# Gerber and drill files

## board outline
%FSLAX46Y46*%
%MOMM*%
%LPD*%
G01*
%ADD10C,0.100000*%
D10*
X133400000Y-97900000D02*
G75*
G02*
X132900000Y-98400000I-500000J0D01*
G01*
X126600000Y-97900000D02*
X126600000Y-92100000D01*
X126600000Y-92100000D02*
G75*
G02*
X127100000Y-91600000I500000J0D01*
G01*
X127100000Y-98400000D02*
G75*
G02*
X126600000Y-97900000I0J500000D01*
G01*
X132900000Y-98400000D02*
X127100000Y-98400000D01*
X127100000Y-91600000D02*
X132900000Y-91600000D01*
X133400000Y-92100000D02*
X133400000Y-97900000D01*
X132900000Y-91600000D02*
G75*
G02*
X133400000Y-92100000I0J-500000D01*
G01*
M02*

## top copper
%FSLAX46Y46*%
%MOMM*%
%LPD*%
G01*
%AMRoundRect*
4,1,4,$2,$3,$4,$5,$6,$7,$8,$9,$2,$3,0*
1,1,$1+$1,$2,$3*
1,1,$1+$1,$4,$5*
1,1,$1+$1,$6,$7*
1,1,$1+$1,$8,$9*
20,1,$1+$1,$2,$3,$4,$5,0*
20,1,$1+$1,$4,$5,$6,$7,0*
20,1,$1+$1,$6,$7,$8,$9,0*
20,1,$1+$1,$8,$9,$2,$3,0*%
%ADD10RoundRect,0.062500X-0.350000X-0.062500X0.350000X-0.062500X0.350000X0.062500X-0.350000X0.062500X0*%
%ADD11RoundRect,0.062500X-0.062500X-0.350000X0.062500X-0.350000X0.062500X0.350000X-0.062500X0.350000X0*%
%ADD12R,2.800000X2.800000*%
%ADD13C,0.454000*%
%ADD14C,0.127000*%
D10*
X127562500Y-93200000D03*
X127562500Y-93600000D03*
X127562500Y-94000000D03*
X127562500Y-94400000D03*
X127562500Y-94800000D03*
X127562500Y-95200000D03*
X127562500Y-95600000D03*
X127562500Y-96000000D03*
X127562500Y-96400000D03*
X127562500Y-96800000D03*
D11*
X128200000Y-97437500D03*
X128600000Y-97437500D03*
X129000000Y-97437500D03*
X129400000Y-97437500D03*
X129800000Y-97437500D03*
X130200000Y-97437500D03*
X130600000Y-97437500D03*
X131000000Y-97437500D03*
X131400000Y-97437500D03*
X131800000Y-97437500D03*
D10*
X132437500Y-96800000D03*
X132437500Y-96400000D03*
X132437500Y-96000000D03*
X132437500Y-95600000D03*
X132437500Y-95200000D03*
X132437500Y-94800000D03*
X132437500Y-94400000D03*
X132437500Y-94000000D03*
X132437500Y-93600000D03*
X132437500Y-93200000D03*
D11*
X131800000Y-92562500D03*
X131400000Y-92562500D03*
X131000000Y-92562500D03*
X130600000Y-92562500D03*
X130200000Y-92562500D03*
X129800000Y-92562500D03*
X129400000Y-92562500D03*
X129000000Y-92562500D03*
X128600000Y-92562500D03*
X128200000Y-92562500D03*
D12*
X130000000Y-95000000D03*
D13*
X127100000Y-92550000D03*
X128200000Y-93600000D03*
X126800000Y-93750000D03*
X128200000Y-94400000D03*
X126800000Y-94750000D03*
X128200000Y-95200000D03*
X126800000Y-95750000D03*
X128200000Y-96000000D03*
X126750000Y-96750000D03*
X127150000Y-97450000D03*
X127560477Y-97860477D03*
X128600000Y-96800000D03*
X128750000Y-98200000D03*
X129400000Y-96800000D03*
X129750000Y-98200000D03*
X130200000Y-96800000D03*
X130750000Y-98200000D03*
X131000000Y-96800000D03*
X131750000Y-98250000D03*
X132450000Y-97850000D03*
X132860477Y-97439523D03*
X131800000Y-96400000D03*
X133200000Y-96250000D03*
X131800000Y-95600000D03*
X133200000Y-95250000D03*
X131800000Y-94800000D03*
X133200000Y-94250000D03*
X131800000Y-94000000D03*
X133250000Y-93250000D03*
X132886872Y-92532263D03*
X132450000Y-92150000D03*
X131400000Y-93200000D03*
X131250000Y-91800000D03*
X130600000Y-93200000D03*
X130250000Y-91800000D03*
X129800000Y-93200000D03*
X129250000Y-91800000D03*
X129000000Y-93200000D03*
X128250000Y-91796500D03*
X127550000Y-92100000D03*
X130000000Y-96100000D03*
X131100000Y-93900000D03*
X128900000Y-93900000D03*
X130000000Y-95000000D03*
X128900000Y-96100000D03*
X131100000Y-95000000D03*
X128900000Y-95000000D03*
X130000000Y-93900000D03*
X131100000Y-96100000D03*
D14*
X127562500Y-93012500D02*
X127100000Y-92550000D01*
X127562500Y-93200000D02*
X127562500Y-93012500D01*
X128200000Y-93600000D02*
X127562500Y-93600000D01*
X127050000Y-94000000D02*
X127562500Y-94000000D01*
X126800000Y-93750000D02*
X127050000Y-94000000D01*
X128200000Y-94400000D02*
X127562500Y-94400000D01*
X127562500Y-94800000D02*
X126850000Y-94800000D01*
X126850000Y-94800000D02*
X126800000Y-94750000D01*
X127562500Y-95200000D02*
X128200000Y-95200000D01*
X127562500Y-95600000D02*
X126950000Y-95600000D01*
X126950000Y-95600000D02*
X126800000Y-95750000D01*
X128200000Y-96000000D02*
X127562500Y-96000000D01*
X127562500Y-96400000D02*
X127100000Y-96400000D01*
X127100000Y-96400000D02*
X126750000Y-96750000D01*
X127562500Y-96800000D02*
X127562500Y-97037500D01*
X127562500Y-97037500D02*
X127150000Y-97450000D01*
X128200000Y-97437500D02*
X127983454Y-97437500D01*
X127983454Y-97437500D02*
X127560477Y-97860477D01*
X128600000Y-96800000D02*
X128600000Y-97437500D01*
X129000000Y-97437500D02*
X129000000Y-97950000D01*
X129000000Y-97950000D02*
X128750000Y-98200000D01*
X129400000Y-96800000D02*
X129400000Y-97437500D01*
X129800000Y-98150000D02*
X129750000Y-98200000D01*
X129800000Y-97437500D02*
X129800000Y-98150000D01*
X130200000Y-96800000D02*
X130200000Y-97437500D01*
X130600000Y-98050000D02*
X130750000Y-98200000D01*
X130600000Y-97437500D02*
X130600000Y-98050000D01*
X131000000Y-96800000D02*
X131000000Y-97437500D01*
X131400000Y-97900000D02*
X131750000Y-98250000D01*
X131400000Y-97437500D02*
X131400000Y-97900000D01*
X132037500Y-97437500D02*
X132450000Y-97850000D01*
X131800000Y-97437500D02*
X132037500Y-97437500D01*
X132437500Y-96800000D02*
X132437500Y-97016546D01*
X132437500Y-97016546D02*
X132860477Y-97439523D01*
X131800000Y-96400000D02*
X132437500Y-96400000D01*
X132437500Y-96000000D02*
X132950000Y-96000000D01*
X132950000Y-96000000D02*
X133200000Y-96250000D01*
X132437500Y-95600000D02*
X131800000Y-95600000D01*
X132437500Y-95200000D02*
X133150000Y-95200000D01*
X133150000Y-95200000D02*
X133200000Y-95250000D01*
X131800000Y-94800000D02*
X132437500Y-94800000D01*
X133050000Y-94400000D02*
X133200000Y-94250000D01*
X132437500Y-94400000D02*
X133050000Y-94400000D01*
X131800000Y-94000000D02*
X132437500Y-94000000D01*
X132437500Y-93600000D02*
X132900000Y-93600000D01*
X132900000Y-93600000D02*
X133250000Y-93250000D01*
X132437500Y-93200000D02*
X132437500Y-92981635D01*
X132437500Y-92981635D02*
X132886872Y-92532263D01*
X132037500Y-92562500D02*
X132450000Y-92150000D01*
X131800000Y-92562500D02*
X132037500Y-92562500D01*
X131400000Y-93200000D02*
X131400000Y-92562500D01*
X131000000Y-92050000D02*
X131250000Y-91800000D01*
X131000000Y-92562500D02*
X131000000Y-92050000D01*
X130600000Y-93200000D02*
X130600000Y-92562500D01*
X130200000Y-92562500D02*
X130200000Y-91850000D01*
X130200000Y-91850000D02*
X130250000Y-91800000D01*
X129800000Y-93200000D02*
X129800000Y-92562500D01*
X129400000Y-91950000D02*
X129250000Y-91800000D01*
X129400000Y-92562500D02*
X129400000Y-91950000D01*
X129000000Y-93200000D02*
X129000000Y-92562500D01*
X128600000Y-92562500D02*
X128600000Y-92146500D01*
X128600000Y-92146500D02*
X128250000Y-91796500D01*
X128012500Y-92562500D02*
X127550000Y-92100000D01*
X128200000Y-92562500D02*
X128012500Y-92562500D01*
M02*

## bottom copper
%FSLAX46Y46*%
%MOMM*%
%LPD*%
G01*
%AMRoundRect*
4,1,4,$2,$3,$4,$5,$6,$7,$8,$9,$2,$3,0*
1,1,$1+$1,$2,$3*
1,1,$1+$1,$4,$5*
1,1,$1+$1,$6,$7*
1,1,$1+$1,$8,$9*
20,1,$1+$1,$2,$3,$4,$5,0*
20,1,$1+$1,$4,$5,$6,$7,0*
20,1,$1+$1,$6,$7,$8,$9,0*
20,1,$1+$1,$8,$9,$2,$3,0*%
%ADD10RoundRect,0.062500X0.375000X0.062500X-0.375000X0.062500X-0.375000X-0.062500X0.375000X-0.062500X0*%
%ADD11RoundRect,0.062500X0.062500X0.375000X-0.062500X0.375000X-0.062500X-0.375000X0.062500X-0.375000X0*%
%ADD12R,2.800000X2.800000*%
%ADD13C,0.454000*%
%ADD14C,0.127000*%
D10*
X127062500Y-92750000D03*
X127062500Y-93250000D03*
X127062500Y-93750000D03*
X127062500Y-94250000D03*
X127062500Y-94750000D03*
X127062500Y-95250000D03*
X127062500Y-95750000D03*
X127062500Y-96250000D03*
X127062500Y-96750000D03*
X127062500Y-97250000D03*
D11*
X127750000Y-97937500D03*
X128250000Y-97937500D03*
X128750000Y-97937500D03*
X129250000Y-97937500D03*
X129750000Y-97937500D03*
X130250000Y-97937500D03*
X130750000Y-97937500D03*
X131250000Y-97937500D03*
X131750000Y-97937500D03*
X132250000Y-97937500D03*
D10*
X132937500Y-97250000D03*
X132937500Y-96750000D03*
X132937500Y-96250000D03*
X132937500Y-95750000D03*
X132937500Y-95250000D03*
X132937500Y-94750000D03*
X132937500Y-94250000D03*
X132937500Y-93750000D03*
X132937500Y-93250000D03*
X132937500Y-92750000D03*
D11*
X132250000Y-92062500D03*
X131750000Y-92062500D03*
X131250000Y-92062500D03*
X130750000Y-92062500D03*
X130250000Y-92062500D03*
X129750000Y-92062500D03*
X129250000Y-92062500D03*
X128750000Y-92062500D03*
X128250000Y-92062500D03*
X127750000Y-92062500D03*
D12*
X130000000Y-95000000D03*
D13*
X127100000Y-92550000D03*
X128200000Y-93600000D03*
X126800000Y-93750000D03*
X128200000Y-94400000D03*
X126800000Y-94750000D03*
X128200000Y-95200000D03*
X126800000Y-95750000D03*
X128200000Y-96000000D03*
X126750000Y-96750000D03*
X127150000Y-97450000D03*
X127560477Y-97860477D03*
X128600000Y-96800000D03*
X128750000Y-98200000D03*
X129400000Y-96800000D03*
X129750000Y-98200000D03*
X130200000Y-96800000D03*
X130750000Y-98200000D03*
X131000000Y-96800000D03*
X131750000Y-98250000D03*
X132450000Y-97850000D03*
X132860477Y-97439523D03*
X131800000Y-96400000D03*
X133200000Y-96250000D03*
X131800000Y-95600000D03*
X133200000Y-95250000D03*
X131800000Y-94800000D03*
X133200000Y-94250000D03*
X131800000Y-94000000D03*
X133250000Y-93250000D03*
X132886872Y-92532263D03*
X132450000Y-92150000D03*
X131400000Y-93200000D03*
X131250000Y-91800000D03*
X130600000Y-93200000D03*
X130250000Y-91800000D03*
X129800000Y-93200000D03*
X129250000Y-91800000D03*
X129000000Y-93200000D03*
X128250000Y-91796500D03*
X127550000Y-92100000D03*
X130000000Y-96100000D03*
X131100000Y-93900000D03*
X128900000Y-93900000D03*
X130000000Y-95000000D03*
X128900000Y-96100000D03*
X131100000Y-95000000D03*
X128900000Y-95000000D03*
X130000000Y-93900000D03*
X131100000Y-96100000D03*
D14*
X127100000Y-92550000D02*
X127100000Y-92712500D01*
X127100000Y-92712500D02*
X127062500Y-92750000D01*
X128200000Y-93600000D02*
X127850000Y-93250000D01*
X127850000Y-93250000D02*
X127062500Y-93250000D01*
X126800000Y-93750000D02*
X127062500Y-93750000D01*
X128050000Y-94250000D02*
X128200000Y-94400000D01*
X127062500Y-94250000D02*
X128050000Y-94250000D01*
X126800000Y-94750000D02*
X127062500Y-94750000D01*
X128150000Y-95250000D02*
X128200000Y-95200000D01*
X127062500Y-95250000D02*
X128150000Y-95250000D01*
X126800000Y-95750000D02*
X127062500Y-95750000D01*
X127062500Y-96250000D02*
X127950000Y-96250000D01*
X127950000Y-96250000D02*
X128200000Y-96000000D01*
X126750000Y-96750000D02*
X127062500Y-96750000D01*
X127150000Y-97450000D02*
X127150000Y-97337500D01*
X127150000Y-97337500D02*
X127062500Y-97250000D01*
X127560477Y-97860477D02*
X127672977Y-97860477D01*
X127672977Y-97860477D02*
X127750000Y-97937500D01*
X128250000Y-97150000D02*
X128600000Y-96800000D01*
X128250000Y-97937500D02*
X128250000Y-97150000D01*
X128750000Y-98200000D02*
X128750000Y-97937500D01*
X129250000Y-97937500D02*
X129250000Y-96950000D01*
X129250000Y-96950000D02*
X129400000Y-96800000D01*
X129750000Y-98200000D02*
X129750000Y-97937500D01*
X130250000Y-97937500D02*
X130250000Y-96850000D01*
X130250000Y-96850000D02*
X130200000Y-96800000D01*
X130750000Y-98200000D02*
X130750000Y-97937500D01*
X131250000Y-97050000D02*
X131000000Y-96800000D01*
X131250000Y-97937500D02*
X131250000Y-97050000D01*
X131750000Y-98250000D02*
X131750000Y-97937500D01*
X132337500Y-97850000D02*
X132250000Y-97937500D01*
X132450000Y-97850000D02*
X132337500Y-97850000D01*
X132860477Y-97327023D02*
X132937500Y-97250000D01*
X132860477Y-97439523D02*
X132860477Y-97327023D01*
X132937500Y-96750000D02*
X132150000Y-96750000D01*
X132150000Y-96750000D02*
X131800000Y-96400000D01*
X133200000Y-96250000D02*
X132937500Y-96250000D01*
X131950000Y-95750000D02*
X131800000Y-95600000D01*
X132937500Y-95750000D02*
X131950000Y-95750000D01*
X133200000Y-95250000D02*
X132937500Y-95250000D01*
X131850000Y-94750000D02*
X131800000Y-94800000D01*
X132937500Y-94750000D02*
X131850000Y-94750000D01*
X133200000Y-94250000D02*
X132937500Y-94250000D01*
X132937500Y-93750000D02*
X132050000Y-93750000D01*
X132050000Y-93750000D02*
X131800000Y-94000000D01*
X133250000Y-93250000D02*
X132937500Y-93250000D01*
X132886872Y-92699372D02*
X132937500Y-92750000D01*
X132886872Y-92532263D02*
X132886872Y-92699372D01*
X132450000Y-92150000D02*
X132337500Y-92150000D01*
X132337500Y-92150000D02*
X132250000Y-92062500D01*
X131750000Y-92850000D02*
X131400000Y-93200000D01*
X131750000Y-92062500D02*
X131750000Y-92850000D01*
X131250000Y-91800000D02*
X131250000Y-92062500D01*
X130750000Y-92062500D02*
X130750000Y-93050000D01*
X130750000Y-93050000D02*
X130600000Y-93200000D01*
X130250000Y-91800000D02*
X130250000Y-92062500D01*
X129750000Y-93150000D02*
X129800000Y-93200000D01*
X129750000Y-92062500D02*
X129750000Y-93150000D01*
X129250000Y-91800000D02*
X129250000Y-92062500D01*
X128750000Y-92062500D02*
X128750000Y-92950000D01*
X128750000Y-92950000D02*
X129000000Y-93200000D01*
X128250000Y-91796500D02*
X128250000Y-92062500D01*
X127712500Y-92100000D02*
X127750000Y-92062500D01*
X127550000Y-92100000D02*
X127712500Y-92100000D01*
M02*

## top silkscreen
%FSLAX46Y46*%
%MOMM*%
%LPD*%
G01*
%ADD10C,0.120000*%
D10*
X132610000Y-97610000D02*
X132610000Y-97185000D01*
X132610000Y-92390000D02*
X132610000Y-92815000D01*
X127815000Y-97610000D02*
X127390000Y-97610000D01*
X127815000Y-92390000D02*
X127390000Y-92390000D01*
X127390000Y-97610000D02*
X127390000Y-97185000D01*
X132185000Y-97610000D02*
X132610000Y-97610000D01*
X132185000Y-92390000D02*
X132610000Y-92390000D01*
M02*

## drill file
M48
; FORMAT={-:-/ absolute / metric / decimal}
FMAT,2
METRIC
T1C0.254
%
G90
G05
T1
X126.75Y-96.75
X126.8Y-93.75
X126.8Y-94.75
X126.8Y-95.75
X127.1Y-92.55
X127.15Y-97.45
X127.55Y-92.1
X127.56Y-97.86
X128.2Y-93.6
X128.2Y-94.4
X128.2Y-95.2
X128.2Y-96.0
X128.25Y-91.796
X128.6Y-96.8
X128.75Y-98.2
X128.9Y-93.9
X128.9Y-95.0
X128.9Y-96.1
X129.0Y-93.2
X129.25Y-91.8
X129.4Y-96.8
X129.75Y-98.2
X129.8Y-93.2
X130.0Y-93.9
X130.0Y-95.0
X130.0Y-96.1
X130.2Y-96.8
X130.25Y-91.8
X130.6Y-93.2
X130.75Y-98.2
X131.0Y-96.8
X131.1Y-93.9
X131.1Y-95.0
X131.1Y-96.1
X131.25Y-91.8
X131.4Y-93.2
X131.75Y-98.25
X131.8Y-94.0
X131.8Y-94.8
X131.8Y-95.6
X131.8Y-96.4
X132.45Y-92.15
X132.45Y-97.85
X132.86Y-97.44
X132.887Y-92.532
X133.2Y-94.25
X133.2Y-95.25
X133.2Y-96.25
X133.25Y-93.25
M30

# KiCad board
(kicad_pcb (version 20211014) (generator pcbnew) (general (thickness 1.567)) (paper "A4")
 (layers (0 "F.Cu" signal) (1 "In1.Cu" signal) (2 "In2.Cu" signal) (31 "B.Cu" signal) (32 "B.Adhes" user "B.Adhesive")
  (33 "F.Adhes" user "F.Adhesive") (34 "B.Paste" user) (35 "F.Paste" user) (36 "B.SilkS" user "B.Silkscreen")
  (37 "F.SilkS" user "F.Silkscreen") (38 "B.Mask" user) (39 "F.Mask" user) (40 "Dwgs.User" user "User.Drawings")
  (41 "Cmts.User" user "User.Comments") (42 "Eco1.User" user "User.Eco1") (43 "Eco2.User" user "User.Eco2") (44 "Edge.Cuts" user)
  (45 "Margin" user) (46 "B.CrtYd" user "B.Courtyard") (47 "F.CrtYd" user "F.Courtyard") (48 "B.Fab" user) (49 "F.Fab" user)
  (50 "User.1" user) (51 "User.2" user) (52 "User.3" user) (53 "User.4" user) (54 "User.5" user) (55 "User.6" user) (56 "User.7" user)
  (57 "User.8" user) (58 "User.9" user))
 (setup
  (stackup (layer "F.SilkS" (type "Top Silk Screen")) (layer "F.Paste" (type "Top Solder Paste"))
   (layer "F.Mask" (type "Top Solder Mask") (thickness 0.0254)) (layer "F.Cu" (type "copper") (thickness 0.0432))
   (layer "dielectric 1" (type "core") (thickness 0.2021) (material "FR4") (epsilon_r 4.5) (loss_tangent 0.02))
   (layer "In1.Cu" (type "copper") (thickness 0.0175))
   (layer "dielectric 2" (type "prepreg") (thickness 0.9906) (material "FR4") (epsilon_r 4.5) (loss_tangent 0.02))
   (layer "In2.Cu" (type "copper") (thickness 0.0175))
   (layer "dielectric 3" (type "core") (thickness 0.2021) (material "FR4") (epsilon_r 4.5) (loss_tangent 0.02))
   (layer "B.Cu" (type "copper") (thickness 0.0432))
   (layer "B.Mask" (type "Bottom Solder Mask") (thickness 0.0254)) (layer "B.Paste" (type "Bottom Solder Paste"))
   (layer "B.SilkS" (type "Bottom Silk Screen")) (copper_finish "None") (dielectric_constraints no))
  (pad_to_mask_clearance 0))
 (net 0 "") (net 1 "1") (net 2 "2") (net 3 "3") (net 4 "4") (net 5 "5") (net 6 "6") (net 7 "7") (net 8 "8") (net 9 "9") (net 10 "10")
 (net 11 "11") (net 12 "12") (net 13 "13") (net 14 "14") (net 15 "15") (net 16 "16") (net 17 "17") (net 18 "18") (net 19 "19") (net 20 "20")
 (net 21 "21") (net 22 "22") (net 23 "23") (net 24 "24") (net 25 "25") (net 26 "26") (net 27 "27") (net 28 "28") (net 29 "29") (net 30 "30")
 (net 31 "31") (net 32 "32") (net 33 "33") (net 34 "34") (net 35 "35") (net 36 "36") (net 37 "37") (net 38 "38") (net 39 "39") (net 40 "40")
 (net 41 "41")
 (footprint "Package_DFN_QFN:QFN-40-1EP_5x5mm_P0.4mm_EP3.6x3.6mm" (layer "F.Cu") (at 130 95)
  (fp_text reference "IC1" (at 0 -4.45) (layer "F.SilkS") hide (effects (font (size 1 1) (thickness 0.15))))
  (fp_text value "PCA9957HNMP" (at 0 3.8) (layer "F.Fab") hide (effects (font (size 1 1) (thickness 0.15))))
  (fp_line (start 2.61 2.61) (end 2.61 2.185) (layer "F.SilkS") (width 0.12))
  (fp_line (start 2.61 -2.61) (end 2.61 -2.185) (layer "F.SilkS") (width 0.12))
  (fp_line (start -2.185 2.61) (end -2.61 2.61) (layer "F.SilkS") (width 0.12))
  (fp_line (start -2.185 -2.61) (end -2.61 -2.61) (layer "F.SilkS") (width 0.12))
  (fp_line (start -2.61 2.61) (end -2.61 2.185) (layer "F.SilkS") (width 0.12))
  (fp_line (start 2.185 2.61) (end 2.61 2.61) (layer "F.SilkS") (width 0.12))
  (fp_line (start 2.185 -2.61) (end 2.61 -2.61) (layer "F.SilkS") (width 0.12))
  (pad "1" smd roundrect (at -2.4375 -1.8) (size 0.825 0.25) (layers "F.Cu" "F.Paste" "F.Mask") (roundrect_rratio 0.25) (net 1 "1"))
  (pad "2" smd roundrect (at -2.4375 -1.4) (size 0.825 0.25) (layers "F.Cu" "F.Paste" "F.Mask") (roundrect_rratio 0.25) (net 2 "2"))
  (pad "3" smd roundrect (at -2.4375 -1) (size 0.825 0.25) (layers "F.Cu" "F.Paste" "F.Mask") (roundrect_rratio 0.25) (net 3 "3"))
  (pad "4" smd roundrect (at -2.4375 -0.6) (size 0.825 0.25) (layers "F.Cu" "F.Paste" "F.Mask") (roundrect_rratio 0.25) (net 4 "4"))
  (pad "5" smd roundrect (at -2.4375 -0.2) (size 0.825 0.25) (layers "F.Cu" "F.Paste" "F.Mask") (roundrect_rratio 0.25) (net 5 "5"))
  (pad "6" smd roundrect (at -2.4375 0.2) (size 0.825 0.25) (layers "F.Cu" "F.Paste" "F.Mask") (roundrect_rratio 0.25) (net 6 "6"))
  (pad "7" smd roundrect (at -2.4375 0.6) (size 0.825 0.25) (layers "F.Cu" "F.Paste" "F.Mask") (roundrect_rratio 0.25) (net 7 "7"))
  (pad "8" smd roundrect (at -2.4375 1) (size 0.825 0.25) (layers "F.Cu" "F.Paste" "F.Mask") (roundrect_rratio 0.25) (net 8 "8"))
  (pad "9" smd roundrect (at -2.4375 1.4) (size 0.825 0.25) (layers "F.Cu" "F.Paste" "F.Mask") (roundrect_rratio 0.25) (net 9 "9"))
  (pad "10" smd roundrect (at -2.4375 1.8) (size 0.825 0.25) (layers "F.Cu" "F.Paste" "F.Mask") (roundrect_rratio 0.25) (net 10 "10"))
  (pad "11" smd roundrect (at -1.8 2.4375) (size 0.25 0.825) (layers "F.Cu" "F.Paste" "F.Mask") (roundrect_rratio 0.25) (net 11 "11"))
  (pad "12" smd roundrect (at -1.4 2.4375) (size 0.25 0.825) (layers "F.Cu" "F.Paste" "F.Mask") (roundrect_rratio 0.25) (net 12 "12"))
  (pad "13" smd roundrect (at -1 2.4375) (size 0.25 0.825) (layers "F.Cu" "F.Paste" "F.Mask") (roundrect_rratio 0.25) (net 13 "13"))
  (pad "14" smd roundrect (at -0.6 2.4375) (size 0.25 0.825) (layers "F.Cu" "F.Paste" "F.Mask") (roundrect_rratio 0.25) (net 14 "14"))
  (pad "15" smd roundrect (at -0.2 2.4375) (size 0.25 0.825) (layers "F.Cu" "F.Paste" "F.Mask") (roundrect_rratio 0.25) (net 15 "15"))
  (pad "16" smd roundrect (at 0.2 2.4375) (size 0.25 0.825) (layers "F.Cu" "F.Paste" "F.Mask") (roundrect_rratio 0.25) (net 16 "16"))
  (pad "17" smd roundrect (at 0.6 2.4375) (size 0.25 0.825) (layers "F.Cu" "F.Paste" "F.Mask") (roundrect_rratio 0.25) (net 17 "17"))
  (pad "18" smd roundrect (at 1 2.4375) (size 0.25 0.825) (layers "F.Cu" "F.Paste" "F.Mask") (roundrect_rratio 0.25) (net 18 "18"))
  (pad "19" smd roundrect (at 1.4 2.4375) (size 0.25 0.825) (layers "F.Cu" "F.Paste" "F.Mask") (roundrect_rratio 0.25) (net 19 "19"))
  (pad "20" smd roundrect (at 1.8 2.4375) (size 0.25 0.825) (layers "F.Cu" "F.Paste" "F.Mask") (roundrect_rratio 0.25) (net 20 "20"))
  (pad "21" smd roundrect (at 2.4375 1.8) (size 0.825 0.25) (layers "F.Cu" "F.Paste" "F.Mask") (roundrect_rratio 0.25) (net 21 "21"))
  (pad "22" smd roundrect (at 2.4375 1.4) (size 0.825 0.25) (layers "F.Cu" "F.Paste" "F.Mask") (roundrect_rratio 0.25) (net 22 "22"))
  (pad "23" smd roundrect (at 2.4375 1) (size 0.825 0.25) (layers "F.Cu" "F.Paste" "F.Mask") (roundrect_rratio 0.25) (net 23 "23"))
  (pad "24" smd roundrect (at 2.4375 0.6) (size 0.825 0.25) (layers "F.Cu" "F.Paste" "F.Mask") (roundrect_rratio 0.25) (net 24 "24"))
  (pad "25" smd roundrect (at 2.4375 0.2) (size 0.825 0.25) (layers "F.Cu" "F.Paste" "F.Mask") (roundrect_rratio 0.25) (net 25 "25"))
  (pad "26" smd roundrect (at 2.4375 -0.2) (size 0.825 0.25) (layers "F.Cu" "F.Paste" "F.Mask") (roundrect_rratio 0.25) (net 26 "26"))
  (pad "27" smd roundrect (at 2.4375 -0.6) (size 0.825 0.25) (layers "F.Cu" "F.Paste" "F.Mask") (roundrect_rratio 0.25) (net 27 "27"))
  (pad "28" smd roundrect (at 2.4375 -1) (size 0.825 0.25) (layers "F.Cu" "F.Paste" "F.Mask") (roundrect_rratio 0.25) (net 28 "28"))
  (pad "29" smd roundrect (at 2.4375 -1.4) (size 0.825 0.25) (layers "F.Cu" "F.Paste" "F.Mask") (roundrect_rratio 0.25) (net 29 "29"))
  (pad "30" smd roundrect (at 2.4375 -1.8) (size 0.825 0.25) (layers "F.Cu" "F.Paste" "F.Mask") (roundrect_rratio 0.25) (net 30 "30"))
  (pad "31" smd roundrect (at 1.8 -2.4375) (size 0.25 0.825) (layers "F.Cu" "F.Paste" "F.Mask") (roundrect_rratio 0.25) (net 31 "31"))
  (pad "32" smd roundrect (at 1.4 -2.4375) (size 0.25 0.825) (layers "F.Cu" "F.Paste" "F.Mask") (roundrect_rratio 0.25) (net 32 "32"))
  (pad "33" smd roundrect (at 1 -2.4375) (size 0.25 0.825) (layers "F.Cu" "F.Paste" "F.Mask") (roundrect_rratio 0.25) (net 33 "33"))
  (pad "34" smd roundrect (at 0.6 -2.4375) (size 0.25 0.825) (layers "F.Cu" "F.Paste" "F.Mask") (roundrect_rratio 0.25) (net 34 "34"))
  (pad "35" smd roundrect (at 0.2 -2.4375) (size 0.25 0.825) (layers "F.Cu" "F.Paste" "F.Mask") (roundrect_rratio 0.25) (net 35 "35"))
  (pad "36" smd roundrect (at -0.2 -2.4375) (size 0.25 0.825) (layers "F.Cu" "F.Paste" "F.Mask") (roundrect_rratio 0.25) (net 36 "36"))
  (pad "37" smd roundrect (at -0.6 -2.4375) (size 0.25 0.825) (layers "F.Cu" "F.Paste" "F.Mask") (roundrect_rratio 0.25) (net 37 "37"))
  (pad "38" smd roundrect (at -1 -2.4375) (size 0.25 0.825) (layers "F.Cu" "F.Paste" "F.Mask") (roundrect_rratio 0.25) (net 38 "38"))
  (pad "39" smd roundrect (at -1.4 -2.4375) (size 0.25 0.825) (layers "F.Cu" "F.Paste" "F.Mask") (roundrect_rratio 0.25) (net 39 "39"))
  (pad "40" smd roundrect (at -1.8 -2.4375) (size 0.25 0.825) (layers "F.Cu" "F.Paste" "F.Mask") (roundrect_rratio 0.25) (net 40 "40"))
  (pad "41" smd rect (at 0 0) (size 2.8 2.8) (layers "F.Cu" "F.Mask") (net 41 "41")))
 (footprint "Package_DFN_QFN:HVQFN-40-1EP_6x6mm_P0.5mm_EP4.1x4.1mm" (layer "B.Cu") (at 130 95 180)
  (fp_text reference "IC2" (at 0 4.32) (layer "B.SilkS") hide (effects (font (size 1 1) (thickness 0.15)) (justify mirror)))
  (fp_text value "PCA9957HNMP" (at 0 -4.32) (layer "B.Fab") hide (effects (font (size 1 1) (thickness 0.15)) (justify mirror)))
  (pad "1" smd roundrect (at 2.9375 2.25 180) (size 0.875 0.25) (layers "B.Cu" "B.Paste" "B.Mask") (roundrect_rratio 0.25) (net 1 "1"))
  (pad "2" smd roundrect (at 2.9375 1.75 180) (size 0.875 0.25) (layers "B.Cu" "B.Paste" "B.Mask") (roundrect_rratio 0.25) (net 2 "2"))
  (pad "3" smd roundrect (at 2.9375 1.25 180) (size 0.875 0.25) (layers "B.Cu" "B.Paste" "B.Mask") (roundrect_rratio 0.25) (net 3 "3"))
  (pad "4" smd roundrect (at 2.9375 0.75 180) (size 0.875 0.25) (layers "B.Cu" "B.Paste" "B.Mask") (roundrect_rratio 0.25) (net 4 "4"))
  (pad "5" smd roundrect (at 2.9375 0.25 180) (size 0.875 0.25) (layers "B.Cu" "B.Paste" "B.Mask") (roundrect_rratio 0.25) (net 5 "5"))
  (pad "6" smd roundrect (at 2.9375 -0.25 180) (size 0.875 0.25) (layers "B.Cu" "B.Paste" "B.Mask") (roundrect_rratio 0.25) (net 6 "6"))
  (pad "7" smd roundrect (at 2.9375 -0.75 180) (size 0.875 0.25) (layers "B.Cu" "B.Paste" "B.Mask") (roundrect_rratio 0.25) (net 7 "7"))
  (pad "8" smd roundrect (at 2.9375 -1.25 180) (size 0.875 0.25) (layers "B.Cu" "B.Paste" "B.Mask") (roundrect_rratio 0.25) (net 8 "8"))
  (pad "9" smd roundrect (at 2.9375 -1.75 180) (size 0.875 0.25) (layers "B.Cu" "B.Paste" "B.Mask") (roundrect_rratio 0.25) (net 9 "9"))
  (pad "10" smd roundrect (at 2.9375 -2.25 180) (size 0.875 0.25) (layers "B.Cu" "B.Paste" "B.Mask") (roundrect_rratio 0.25) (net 10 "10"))
  (pad "11" smd roundrect (at 2.25 -2.9375 180) (size 0.25 0.875) (layers "B.Cu" "B.Paste" "B.Mask") (roundrect_rratio 0.25) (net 11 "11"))
  (pad "12" smd roundrect (at 1.75 -2.9375 180) (size 0.25 0.875) (layers "B.Cu" "B.Paste" "B.Mask") (roundrect_rratio 0.25) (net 12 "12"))
  (pad "13" smd roundrect (at 1.25 -2.9375 180) (size 0.25 0.875) (layers "B.Cu" "B.Paste" "B.Mask") (roundrect_rratio 0.25) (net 13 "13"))
  (pad "14" smd roundrect (at 0.75 -2.9375 180) (size 0.25 0.875) (layers "B.Cu" "B.Paste" "B.Mask") (roundrect_rratio 0.25) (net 14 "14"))
  (pad "15" smd roundrect (at 0.25 -2.9375 180) (size 0.25 0.875) (layers "B.Cu" "B.Paste" "B.Mask") (roundrect_rratio 0.25) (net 15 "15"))
  (pad "16" smd roundrect (at -0.25 -2.9375 180) (size 0.25 0.875) (layers "B.Cu" "B.Paste" "B.Mask") (roundrect_rratio 0.25) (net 16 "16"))
  (pad "17" smd roundrect (at -0.75 -2.9375 180) (size 0.25 0.875) (layers "B.Cu" "B.Paste" "B.Mask") (roundrect_rratio 0.25) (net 17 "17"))
  (pad "18" smd roundrect (at -1.25 -2.9375 180) (size 0.25 0.875) (layers "B.Cu" "B.Paste" "B.Mask") (roundrect_rratio 0.25) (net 18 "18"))
  (pad "19" smd roundrect (at -1.75 -2.9375 180) (size 0.25 0.875) (layers "B.Cu" "B.Paste" "B.Mask") (roundrect_rratio 0.25) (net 19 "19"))
  (pad "20" smd roundrect (at -2.25 -2.9375 180) (size 0.25 0.875) (layers "B.Cu" "B.Paste" "B.Mask") (roundrect_rratio 0.25) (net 20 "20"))
  (pad "21" smd roundrect (at -2.9375 -2.25 180) (size 0.875 0.25) (layers "B.Cu" "B.Paste" "B.Mask") (roundrect_rratio 0.25) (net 21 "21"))
  (pad "22" smd roundrect (at -2.9375 -1.75 180) (size 0.875 0.25) (layers "B.Cu" "B.Paste" "B.Mask") (roundrect_rratio 0.25) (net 22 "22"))
  (pad "23" smd roundrect (at -2.9375 -1.25 180) (size 0.875 0.25) (layers "B.Cu" "B.Paste" "B.Mask") (roundrect_rratio 0.25) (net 23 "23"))
  (pad "24" smd roundrect (at -2.9375 -0.75 180) (size 0.875 0.25) (layers "B.Cu" "B.Paste" "B.Mask") (roundrect_rratio 0.25) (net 24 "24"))
  (pad "25" smd roundrect (at -2.9375 -0.25 180) (size 0.875 0.25) (layers "B.Cu" "B.Paste" "B.Mask") (roundrect_rratio 0.25) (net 25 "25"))
  (pad "26" smd roundrect (at -2.9375 0.25 180) (size 0.875 0.25) (layers "B.Cu" "B.Paste" "B.Mask") (roundrect_rratio 0.25) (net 26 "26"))
  (pad "27" smd roundrect (at -2.9375 0.75 180) (size 0.875 0.25) (layers "B.Cu" "B.Paste" "B.Mask") (roundrect_rratio 0.25) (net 27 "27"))
  (pad "28" smd roundrect (at -2.9375 1.25 180) (size 0.875 0.25) (layers "B.Cu" "B.Paste" "B.Mask") (roundrect_rratio 0.25) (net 28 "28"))
  (pad "29" smd roundrect (at -2.9375 1.75 180) (size 0.875 0.25) (layers "B.Cu" "B.Paste" "B.Mask") (roundrect_rratio 0.25) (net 29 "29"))
  (pad "30" smd roundrect (at -2.9375 2.25 180) (size 0.875 0.25) (layers "B.Cu" "B.Paste" "B.Mask") (roundrect_rratio 0.25) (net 30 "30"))
  (pad "31" smd roundrect (at -2.25 2.9375 180) (size 0.25 0.875) (layers "B.Cu" "B.Paste" "B.Mask") (roundrect_rratio 0.25) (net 31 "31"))
  (pad "32" smd roundrect (at -1.75 2.9375 180) (size 0.25 0.875) (layers "B.Cu" "B.Paste" "B.Mask") (roundrect_rratio 0.25) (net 32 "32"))
  (pad "33" smd roundrect (at -1.25 2.9375 180) (size 0.25 0.875) (layers "B.Cu" "B.Paste" "B.Mask") (roundrect_rratio 0.25) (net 33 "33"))
  (pad "34" smd roundrect (at -0.75 2.9375 180) (size 0.25 0.875) (layers "B.Cu" "B.Paste" "B.Mask") (roundrect_rratio 0.25) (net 34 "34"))
  (pad "35" smd roundrect (at -0.25 2.9375 180) (size 0.25 0.875) (layers "B.Cu" "B.Paste" "B.Mask") (roundrect_rratio 0.25) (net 35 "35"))
  (pad "36" smd roundrect (at 0.25 2.9375 180) (size 0.25 0.875) (layers "B.Cu" "B.Paste" "B.Mask") (roundrect_rratio 0.25) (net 36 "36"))
  (pad "37" smd roundrect (at 0.75 2.9375 180) (size 0.25 0.875) (layers "B.Cu" "B.Paste" "B.Mask") (roundrect_rratio 0.25) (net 37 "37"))
  (pad "38" smd roundrect (at 1.25 2.9375 180) (size 0.25 0.875) (layers "B.Cu" "B.Paste" "B.Mask") (roundrect_rratio 0.25) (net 38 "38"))
  (pad "39" smd roundrect (at 1.75 2.9375 180) (size 0.25 0.875) (layers "B.Cu" "B.Paste" "B.Mask") (roundrect_rratio 0.25) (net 39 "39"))
  (pad "40" smd roundrect (at 2.25 2.9375 180) (size 0.25 0.875) (layers "B.Cu" "B.Paste" "B.Mask") (roundrect_rratio 0.25) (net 40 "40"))
  (pad "41" smd rect (at 0 0 180) (size 2.8 2.8) (layers "B.Cu" "B.Mask") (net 41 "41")))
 (gr_arc (start 133.4 97.9) (mid 133.253553 98.253553) (end 132.9 98.4) (layer "Edge.Cuts") (width 0.1))
 (gr_line (start 126.6 97.9) (end 126.6 92.1) (layer "Edge.Cuts") (width 0.1))
 (gr_arc (start 126.6 92.1) (mid 126.746447 91.746447) (end 127.1 91.6) (layer "Edge.Cuts") (width 0.1))
 (gr_arc (start 127.1 98.4) (mid 126.746447 98.253553) (end 126.6 97.9) (layer "Edge.Cuts") (width 0.1))
 (gr_line (start 132.9 98.4) (end 127.1 98.4) (layer "Edge.Cuts") (width 0.1))
 (gr_line (start 127.1 91.6) (end 132.9 91.6) (layer "Edge.Cuts") (width 0.1))
 (gr_line (start 133.4 92.1) (end 133.4 97.9) (layer "Edge.Cuts") (width 0.1))
 (gr_arc (start 132.9 91.6) (mid 133.253553 91.746447) (end 133.4 92.1) (layer "Edge.Cuts") (width 0.1))
 (segment (start 127.5625 93.0125) (end 127.1 92.55) (width 0.127) (layer "F.Cu") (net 1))
 (segment (start 127.5625 93.2) (end 127.5625 93.0125) (width 0.127) (layer "F.Cu") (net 1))
 (via (at 127.1 92.55) (size 0.454) (drill 0.254) (layers "F.Cu" "B.Cu") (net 1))
 (segment (start 127.1 92.55) (end 127.1 92.7125) (width 0.127) (layer "B.Cu") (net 1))
 (segment (start 127.1 92.7125) (end 127.0625 92.75) (width 0.127) (layer "B.Cu") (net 1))
 (segment (start 128.2 93.6) (end 127.5625 93.6) (width 0.127) (layer "F.Cu") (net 2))
 (via (at 128.2 93.6) (size 0.454) (drill 0.254) (layers "F.Cu" "B.Cu") (free) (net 2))
 (segment (start 128.2 93.6) (end 127.85 93.25) (width 0.127) (layer "B.Cu") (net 2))
 (segment (start 127.85 93.25) (end 127.0625 93.25) (width 0.127) (layer "B.Cu") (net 2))
 (segment (start 127.05 94) (end 127.5625 94) (width 0.127) (layer "F.Cu") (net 3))
 (segment (start 126.8 93.75) (end 127.05 94) (width 0.127) (layer "F.Cu") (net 3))
 (via (at 126.8 93.75) (size 0.454) (drill 0.254) (layers "F.Cu" "B.Cu") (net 3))
 (segment (start 126.8 93.75) (end 127.0625 93.75) (width 0.127) (layer "B.Cu") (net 3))
 (segment (start 128.2 94.4) (end 127.5625 94.4) (width 0.127) (layer "F.Cu") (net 4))
 (via (at 128.2 94.4) (size 0.454) (drill 0.254) (layers "F.Cu" "B.Cu") (free) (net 4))
 (segment (start 128.05 94.25) (end 128.2 94.4) (width 0.127) (layer "B.Cu") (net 4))
 (segment (start 127.0625 94.25) (end 128.05 94.25) (width 0.127) (layer "B.Cu") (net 4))
 (segment (start 127.5625 94.8) (end 126.85 94.8) (width 0.127) (layer "F.Cu") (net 5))
 (segment (start 126.85 94.8) (end 126.8 94.75) (width 0.127) (layer "F.Cu") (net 5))
 (via (at 126.8 94.75) (size 0.454) (drill 0.254) (layers "F.Cu" "B.Cu") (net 5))
 (segment (start 126.8 94.75) (end 127.0625 94.75) (width 0.127) (layer "B.Cu") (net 5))
 (segment (start 127.5625 95.2) (end 128.2 95.2) (width 0.127) (layer "F.Cu") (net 6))
 (via (at 128.2 95.2) (size 0.454) (drill 0.254) (layers "F.Cu" "B.Cu") (free) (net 6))
 (segment (start 128.15 95.25) (end 128.2 95.2) (width 0.127) (layer "B.Cu") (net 6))
 (segment (start 127.0625 95.25) (end 128.15 95.25) (width 0.127) (layer "B.Cu") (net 6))
 (segment (start 127.5625 95.6) (end 126.95 95.6) (width 0.127) (layer "F.Cu") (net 7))
 (segment (start 126.95 95.6) (end 126.8 95.75) (width 0.127) (layer "F.Cu") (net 7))
 (via (at 126.8 95.75) (size 0.454) (drill 0.254) (layers "F.Cu" "B.Cu") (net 7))
 (segment (start 126.8 95.75) (end 127.0625 95.75) (width 0.127) (layer "B.Cu") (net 7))
 (segment (start 128.2 96) (end 127.5625 96) (width 0.127) (layer "F.Cu") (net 8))
 (via (at 128.2 96) (size 0.454) (drill 0.254) (layers "F.Cu" "B.Cu") (free) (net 8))
 (segment (start 127.0625 96.25) (end 127.95 96.25) (width 0.127) (layer "B.Cu") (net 8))
 (segment (start 127.95 96.25) (end 128.2 96) (width 0.127) (layer "B.Cu") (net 8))
 (segment (start 127.5625 96.4) (end 127.1 96.4) (width 0.127) (layer "F.Cu") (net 9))
 (segment (start 127.1 96.4) (end 126.75 96.75) (width 0.127) (layer "F.Cu") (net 9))
 (via (at 126.75 96.75) (size 0.454) (drill 0.254) (layers "F.Cu" "B.Cu") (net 9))
 (segment (start 126.75 96.75) (end 127.0625 96.75) (width 0.127) (layer "B.Cu") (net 9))
 (segment (start 127.5625 96.8) (end 127.5625 97.0375) (width 0.127) (layer "F.Cu") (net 10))
 (segment (start 127.5625 97.0375) (end 127.15 97.45) (width 0.127) (layer "F.Cu") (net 10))
 (via (at 127.15 97.45) (size 0.454) (drill 0.254) (layers "F.Cu" "B.Cu") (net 10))
 (segment (start 127.15 97.45) (end 127.15 97.3375) (width 0.127) (layer "B.Cu") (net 10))
 (segment (start 127.15 97.3375) (end 127.0625 97.25) (width 0.127) (layer "B.Cu") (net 10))
 (segment (start 128.2 97.4375) (end 127.983454 97.4375) (width 0.127) (layer "F.Cu") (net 11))
 (segment (start 127.983454 97.4375) (end 127.560477 97.860477) (width 0.127) (layer "F.Cu") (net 11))
 (via (at 127.560477 97.860477) (size 0.454) (drill 0.254) (layers "F.Cu" "B.Cu") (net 11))
 (segment (start 127.560477 97.860477) (end 127.672977 97.860477) (width 0.127) (layer "B.Cu") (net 11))
 (segment (start 127.672977 97.860477) (end 127.75 97.9375) (width 0.127) (layer "B.Cu") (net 11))
 (segment (start 128.6 96.8) (end 128.6 97.4375) (width 0.127) (layer "F.Cu") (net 12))
 (via (at 128.6 96.8) (size 0.454) (drill 0.254) (layers "F.Cu" "B.Cu") (free) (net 12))
 (segment (start 128.25 97.15) (end 128.6 96.8) (width 0.127) (layer "B.Cu") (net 12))
 (segment (start 128.25 97.9375) (end 128.25 97.15) (width 0.127) (layer "B.Cu") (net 12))
 (segment (start 129 97.4375) (end 129 97.95) (width 0.127) (layer "F.Cu") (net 13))
 (segment (start 129 97.95) (end 128.75 98.2) (width 0.127) (layer "F.Cu") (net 13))
 (via (at 128.75 98.2) (size 0.454) (drill 0.254) (layers "F.Cu" "B.Cu") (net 13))
 (segment (start 128.75 98.2) (end 128.75 97.9375) (width 0.127) (layer "B.Cu") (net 13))
 (segment (start 129.4 96.8) (end 129.4 97.4375) (width 0.127) (layer "F.Cu") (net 14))
 (via (at 129.4 96.8) (size 0.454) (drill 0.254) (layers "F.Cu" "B.Cu") (free) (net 14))
 (segment (start 129.25 97.9375) (end 129.25 96.95) (width 0.127) (layer "B.Cu") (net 14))
 (segment (start 129.25 96.95) (end 129.4 96.8) (width 0.127) (layer "B.Cu") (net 14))
 (segment (start 129.8 98.15) (end 129.75 98.2) (width 0.127) (layer "F.Cu") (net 15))
 (segment (start 129.8 97.4375) (end 129.8 98.15) (width 0.127) (layer "F.Cu") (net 15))
 (via (at 129.75 98.2) (size 0.454) (drill 0.254) (layers "F.Cu" "B.Cu") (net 15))
 (segment (start 129.75 98.2) (end 129.75 97.9375) (width 0.127) (layer "B.Cu") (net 15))
 (segment (start 130.2 96.8) (end 130.2 97.4375) (width 0.127) (layer "F.Cu") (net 16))
 (via (at 130.2 96.8) (size 0.454) (drill 0.254) (layers "F.Cu" "B.Cu") (free) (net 16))
 (segment (start 130.25 97.9375) (end 130.25 96.85) (width 0.127) (layer "B.Cu") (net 16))
 (segment (start 130.25 96.85) (end 130.2 96.8) (width 0.127) (layer "B.Cu") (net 16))
 (segment (start 130.6 98.05) (end 130.75 98.2) (width 0.127) (layer "F.Cu") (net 17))
 (segment (start 130.6 97.4375) (end 130.6 98.05) (width 0.127) (layer "F.Cu") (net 17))
 (via (at 130.75 98.2) (size 0.454) (drill 0.254) (layers "F.Cu" "B.Cu") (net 17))
 (segment (start 130.75 98.2) (end 130.75 97.9375) (width 0.127) (layer "B.Cu") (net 17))
 (segment (start 131 96.8) (end 131 97.4375) (width 0.127) (layer "F.Cu") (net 18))
 (via (at 131 96.8) (size 0.454) (drill 0.254) (layers "F.Cu" "B.Cu") (free) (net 18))
 (segment (start 131.25 97.05) (end 131 96.8) (width 0.127) (layer "B.Cu") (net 18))
 (segment (start 131.25 97.9375) (end 131.25 97.05) (width 0.127) (layer "B.Cu") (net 18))
 (segment (start 131.4 97.9) (end 131.75 98.25) (width 0.127) (layer "F.Cu") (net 19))
 (segment (start 131.4 97.4375) (end 131.4 97.9) (width 0.127) (layer "F.Cu") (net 19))
 (via (at 131.75 98.25) (size 0.454) (drill 0.254) (layers "F.Cu" "B.Cu") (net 19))
 (segment (start 131.75 98.25) (end 131.75 97.9375) (width 0.127) (layer "B.Cu") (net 19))
 (segment (start 132.0375 97.4375) (end 132.45 97.85) (width 0.127) (layer "F.Cu") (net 20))
 (segment (start 131.8 97.4375) (end 132.0375 97.4375) (width 0.127) (layer "F.Cu") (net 20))
 (via (at 132.45 97.85) (size 0.454) (drill 0.254) (layers "F.Cu" "B.Cu") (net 20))
 (segment (start 132.3375 97.85) (end 132.25 97.9375) (width 0.127) (layer "B.Cu") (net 20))
 (segment (start 132.45 97.85) (end 132.3375 97.85) (width 0.127) (layer "B.Cu") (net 20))
 (segment (start 132.4375 96.8) (end 132.4375 97.016546) (width 0.127) (layer "F.Cu") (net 21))
 (segment (start 132.4375 97.016546) (end 132.860477 97.439523) (width 0.127) (layer "F.Cu") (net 21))
 (via (at 132.860477 97.439523) (size 0.454) (drill 0.254) (layers "F.Cu" "B.Cu") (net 21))
 (segment (start 132.860477 97.327023) (end 132.9375 97.25) (width 0.127) (layer "B.Cu") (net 21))
 (segment (start 132.860477 97.439523) (end 132.860477 97.327023) (width 0.127) (layer "B.Cu") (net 21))
 (segment (start 131.8 96.4) (end 132.4375 96.4) (width 0.127) (layer "F.Cu") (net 22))
 (via (at 131.8 96.4) (size 0.454) (drill 0.254) (layers "F.Cu" "B.Cu") (free) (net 22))
 (segment (start 132.9375 96.75) (end 132.15 96.75) (width 0.127) (layer "B.Cu") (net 22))
 (segment (start 132.15 96.75) (end 131.8 96.4) (width 0.127) (layer "B.Cu") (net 22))
 (segment (start 132.4375 96) (end 132.95 96) (width 0.127) (layer "F.Cu") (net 23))
 (segment (start 132.95 96) (end 133.2 96.25) (width 0.127) (layer "F.Cu") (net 23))
 (via (at 133.2 96.25) (size 0.454) (drill 0.254) (layers "F.Cu" "B.Cu") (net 23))
 (segment (start 133.2 96.25) (end 132.9375 96.25) (width 0.127) (layer "B.Cu") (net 23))
 (segment (start 132.4375 95.6) (end 131.8 95.6) (width 0.127) (layer "F.Cu") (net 24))
 (via (at 131.8 95.6) (size 0.454) (drill 0.254) (layers "F.Cu" "B.Cu") (free) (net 24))
 (segment (start 131.95 95.75) (end 131.8 95.6) (width 0.127) (layer "B.Cu") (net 24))
 (segment (start 132.9375 95.75) (end 131.95 95.75) (width 0.127) (layer "B.Cu") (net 24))
 (segment (start 132.4375 95.2) (end 133.15 95.2) (width 0.127) (layer "F.Cu") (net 25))
 (segment (start 133.15 95.2) (end 133.2 95.25) (width 0.127) (layer "F.Cu") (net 25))
 (via (at 133.2 95.25) (size 0.454) (drill 0.254) (layers "F.Cu" "B.Cu") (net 25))
 (segment (start 133.2 95.25) (end 132.9375 95.25) (width 0.127) (layer "B.Cu") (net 25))
 (segment (start 131.8 94.8) (end 132.4375 94.8) (width 0.127) (layer "F.Cu") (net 26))
 (via (at 131.8 94.8) (size 0.454) (drill 0.254) (layers "F.Cu" "B.Cu") (free) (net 26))
 (segment (start 131.85 94.75) (end 131.8 94.8) (width 0.127) (layer "B.Cu") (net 26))
 (segment (start 132.9375 94.75) (end 131.85 94.75) (width 0.127) (layer "B.Cu") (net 26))
 (segment (start 133.05 94.4) (end 133.2 94.25) (width 0.127) (layer "F.Cu") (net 27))
 (segment (start 132.4375 94.4) (end 133.05 94.4) (width 0.127) (layer "F.Cu") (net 27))
 (via (at 133.2 94.25) (size 0.454) (drill 0.254) (layers "F.Cu" "B.Cu") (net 27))
 (segment (start 133.2 94.25) (end 132.9375 94.25) (width 0.127) (layer "B.Cu") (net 27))
 (segment (start 131.8 94) (end 132.4375 94) (width 0.127) (layer "F.Cu") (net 28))
 (via (at 131.8 94) (size 0.454) (drill 0.254) (layers "F.Cu" "B.Cu") (free) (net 28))
 (segment (start 132.9375 93.75) (end 132.05 93.75) (width 0.127) (layer "B.Cu") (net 28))
 (segment (start 132.05 93.75) (end 131.8 94) (width 0.127) (layer "B.Cu") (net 28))
 (segment (start 132.4375 93.6) (end 132.9 93.6) (width 0.127) (layer "F.Cu") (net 29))
 (segment (start 132.9 93.6) (end 133.25 93.25) (width 0.127) (layer "F.Cu") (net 29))
 (via (at 133.25 93.25) (size 0.454) (drill 0.254) (layers "F.Cu" "B.Cu") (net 29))
 (segment (start 133.25 93.25) (end 132.9375 93.25) (width 0.127) (layer "B.Cu") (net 29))
 (segment (start 132.4375 93.2) (end 132.4375 92.981635) (width 0.127) (layer "F.Cu") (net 30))
 (segment (start 132.4375 92.981635) (end 132.886872 92.532263) (width 0.127) (layer "F.Cu") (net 30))
 (via (at 132.886872 92.532263) (size 0.454) (drill 0.254) (layers "F.Cu" "B.Cu") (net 30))
 (segment (start 132.886872 92.699372) (end 132.9375 92.75) (width 0.127) (layer "B.Cu") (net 30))
 (segment (start 132.886872 92.532263) (end 132.886872 92.699372) (width 0.127) (layer "B.Cu") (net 30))
 (segment (start 132.0375 92.5625) (end 132.45 92.15) (width 0.127) (layer "F.Cu") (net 31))
 (segment (start 131.8 92.5625) (end 132.0375 92.5625) (width 0.127) (layer "F.Cu") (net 31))
 (via (at 132.45 92.15) (size 0.454) (drill 0.254) (layers "F.Cu" "B.Cu") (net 31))
 (segment (start 132.45 92.15) (end 132.3375 92.15) (width 0.127) (layer "B.Cu") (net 31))
 (segment (start 132.3375 92.15) (end 132.25 92.0625) (width 0.127) (layer "B.Cu") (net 31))
 (segment (start 131.4 93.2) (end 131.4 92.5625) (width 0.127) (layer "F.Cu") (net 32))
 (via (at 131.4 93.2) (size 0.454) (drill 0.254) (layers "F.Cu" "B.Cu") (free) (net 32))
 (segment (start 131.75 92.85) (end 131.4 93.2) (width 0.127) (layer "B.Cu") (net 32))
 (segment (start 131.75 92.0625) (end 131.75 92.85) (width 0.127) (layer "B.Cu") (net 32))
 (segment (start 131 92.05) (end 131.25 91.8) (width 0.127) (layer "F.Cu") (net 33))
 (segment (start 131 92.5625) (end 131 92.05) (width 0.127) (layer "F.Cu") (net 33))
 (via (at 131.25 91.8) (size 0.454) (drill 0.254) (layers "F.Cu" "B.Cu") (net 33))
 (segment (start 131.25 91.8) (end 131.25 92.0625) (width 0.127) (layer "B.Cu") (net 33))
 (segment (start 130.6 93.2) (end 130.6 92.5625) (width 0.127) (layer "F.Cu") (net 34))
 (via (at 130.6 93.2) (size 0.454) (drill 0.254) (layers "F.Cu" "B.Cu") (free) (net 34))
 (segment (start 130.75 92.0625) (end 130.75 93.05) (width 0.127) (layer "B.Cu") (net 34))
 (segment (start 130.75 93.05) (end 130.6 93.2) (width 0.127) (layer "B.Cu") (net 34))
 (segment (start 130.2 92.5625) (end 130.2 91.85) (width 0.127) (layer "F.Cu") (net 35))
 (segment (start 130.2 91.85) (end 130.25 91.8) (width 0.127) (layer "F.Cu") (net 35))
 (via (at 130.25 91.8) (size 0.454) (drill 0.254) (layers "F.Cu" "B.Cu") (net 35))
 (segment (start 130.25 91.8) (end 130.25 92.0625) (width 0.127) (layer "B.Cu") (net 35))
 (segment (start 129.8 93.2) (end 129.8 92.5625) (width 0.127) (layer "F.Cu") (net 36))
 (via (at 129.8 93.2) (size 0.454) (drill 0.254) (layers "F.Cu" "B.Cu") (free) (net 36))
 (segment (start 129.75 93.15) (end 129.8 93.2) (width 0.127) (layer "B.Cu") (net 36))
 (segment (start 129.75 92.0625) (end 129.75 93.15) (width 0.127) (layer "B.Cu") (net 36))
 (segment (start 129.4 91.95) (end 129.25 91.8) (width 0.127) (layer "F.Cu") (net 37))
 (segment (start 129.4 92.5625) (end 129.4 91.95) (width 0.127) (layer "F.Cu") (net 37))
 (via (at 129.25 91.8) (size 0.454) (drill 0.254) (layers "F.Cu" "B.Cu") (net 37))
 (segment (start 129.25 91.8) (end 129.25 92.0625) (width 0.127) (layer "B.Cu") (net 37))
 (segment (start 129 93.2) (end 129 92.5625) (width 0.127) (layer "F.Cu") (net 38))
 (via (at 129 93.2) (size 0.454) (drill 0.254) (layers "F.Cu" "B.Cu") (free) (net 38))
 (segment (start 128.75 92.0625) (end 128.75 92.95) (width 0.127) (layer "B.Cu") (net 38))
 (segment (start 128.75 92.95) (end 129 93.2) (width 0.127) (layer "B.Cu") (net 38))
 (segment (start 128.6 92.5625) (end 128.6 92.1465) (width 0.127) (layer "F.Cu") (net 39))
 (segment (start 128.6 92.1465) (end 128.25 91.7965) (width 0.127) (layer "F.Cu") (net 39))
 (via (at 128.25 91.7965) (size 0.454) (drill 0.254) (layers "F.Cu" "B.Cu") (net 39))
 (segment (start 128.25 91.7965) (end 128.25 92.0625) (width 0.127) (layer "B.Cu") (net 39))
 (segment (start 128.0125 92.5625) (end 127.55 92.1) (width 0.127) (layer "F.Cu") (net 40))
 (segment (start 128.2 92.5625) (end 128.0125 92.5625) (width 0.127) (layer "F.Cu") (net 40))
 (via (at 127.55 92.1) (size 0.454) (drill 0.254) (layers "F.Cu" "B.Cu") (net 40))
 (segment (start 127.7125 92.1) (end 127.75 92.0625) (width 0.127) (layer "B.Cu") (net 40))
 (segment (start 127.55 92.1) (end 127.7125 92.1) (width 0.127) (layer "B.Cu") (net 40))
 (via (at 130 96.1) (size 0.454) (drill 0.254) (layers "F.Cu" "B.Cu") (free) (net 41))
 (via (at 131.1 93.9) (size 0.454) (drill 0.254) (layers "F.Cu" "B.Cu") (free) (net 41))
 (via (at 128.9 93.9) (size 0.454) (drill 0.254) (layers "F.Cu" "B.Cu") (free) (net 41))
 (via (at 130 95) (size 0.454) (drill 0.254) (layers "F.Cu" "B.Cu") (free) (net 41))
 (via (at 128.9 96.1) (size 0.454) (drill 0.254) (layers "F.Cu" "B.Cu") (free) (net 41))
 (via (at 131.1 95) (size 0.454) (drill 0.254) (layers "F.Cu" "B.Cu") (free) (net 41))
 (via (at 128.9 95) (size 0.454) (drill 0.254) (layers "F.Cu" "B.Cu") (free) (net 41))
 (via (at 130 93.9) (size 0.454) (drill 0.254) (layers "F.Cu" "B.Cu") (free) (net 41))
 (via (at 131.1 96.1) (size 0.454) (drill 0.254) (layers "F.Cu" "B.Cu") (free) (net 41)))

